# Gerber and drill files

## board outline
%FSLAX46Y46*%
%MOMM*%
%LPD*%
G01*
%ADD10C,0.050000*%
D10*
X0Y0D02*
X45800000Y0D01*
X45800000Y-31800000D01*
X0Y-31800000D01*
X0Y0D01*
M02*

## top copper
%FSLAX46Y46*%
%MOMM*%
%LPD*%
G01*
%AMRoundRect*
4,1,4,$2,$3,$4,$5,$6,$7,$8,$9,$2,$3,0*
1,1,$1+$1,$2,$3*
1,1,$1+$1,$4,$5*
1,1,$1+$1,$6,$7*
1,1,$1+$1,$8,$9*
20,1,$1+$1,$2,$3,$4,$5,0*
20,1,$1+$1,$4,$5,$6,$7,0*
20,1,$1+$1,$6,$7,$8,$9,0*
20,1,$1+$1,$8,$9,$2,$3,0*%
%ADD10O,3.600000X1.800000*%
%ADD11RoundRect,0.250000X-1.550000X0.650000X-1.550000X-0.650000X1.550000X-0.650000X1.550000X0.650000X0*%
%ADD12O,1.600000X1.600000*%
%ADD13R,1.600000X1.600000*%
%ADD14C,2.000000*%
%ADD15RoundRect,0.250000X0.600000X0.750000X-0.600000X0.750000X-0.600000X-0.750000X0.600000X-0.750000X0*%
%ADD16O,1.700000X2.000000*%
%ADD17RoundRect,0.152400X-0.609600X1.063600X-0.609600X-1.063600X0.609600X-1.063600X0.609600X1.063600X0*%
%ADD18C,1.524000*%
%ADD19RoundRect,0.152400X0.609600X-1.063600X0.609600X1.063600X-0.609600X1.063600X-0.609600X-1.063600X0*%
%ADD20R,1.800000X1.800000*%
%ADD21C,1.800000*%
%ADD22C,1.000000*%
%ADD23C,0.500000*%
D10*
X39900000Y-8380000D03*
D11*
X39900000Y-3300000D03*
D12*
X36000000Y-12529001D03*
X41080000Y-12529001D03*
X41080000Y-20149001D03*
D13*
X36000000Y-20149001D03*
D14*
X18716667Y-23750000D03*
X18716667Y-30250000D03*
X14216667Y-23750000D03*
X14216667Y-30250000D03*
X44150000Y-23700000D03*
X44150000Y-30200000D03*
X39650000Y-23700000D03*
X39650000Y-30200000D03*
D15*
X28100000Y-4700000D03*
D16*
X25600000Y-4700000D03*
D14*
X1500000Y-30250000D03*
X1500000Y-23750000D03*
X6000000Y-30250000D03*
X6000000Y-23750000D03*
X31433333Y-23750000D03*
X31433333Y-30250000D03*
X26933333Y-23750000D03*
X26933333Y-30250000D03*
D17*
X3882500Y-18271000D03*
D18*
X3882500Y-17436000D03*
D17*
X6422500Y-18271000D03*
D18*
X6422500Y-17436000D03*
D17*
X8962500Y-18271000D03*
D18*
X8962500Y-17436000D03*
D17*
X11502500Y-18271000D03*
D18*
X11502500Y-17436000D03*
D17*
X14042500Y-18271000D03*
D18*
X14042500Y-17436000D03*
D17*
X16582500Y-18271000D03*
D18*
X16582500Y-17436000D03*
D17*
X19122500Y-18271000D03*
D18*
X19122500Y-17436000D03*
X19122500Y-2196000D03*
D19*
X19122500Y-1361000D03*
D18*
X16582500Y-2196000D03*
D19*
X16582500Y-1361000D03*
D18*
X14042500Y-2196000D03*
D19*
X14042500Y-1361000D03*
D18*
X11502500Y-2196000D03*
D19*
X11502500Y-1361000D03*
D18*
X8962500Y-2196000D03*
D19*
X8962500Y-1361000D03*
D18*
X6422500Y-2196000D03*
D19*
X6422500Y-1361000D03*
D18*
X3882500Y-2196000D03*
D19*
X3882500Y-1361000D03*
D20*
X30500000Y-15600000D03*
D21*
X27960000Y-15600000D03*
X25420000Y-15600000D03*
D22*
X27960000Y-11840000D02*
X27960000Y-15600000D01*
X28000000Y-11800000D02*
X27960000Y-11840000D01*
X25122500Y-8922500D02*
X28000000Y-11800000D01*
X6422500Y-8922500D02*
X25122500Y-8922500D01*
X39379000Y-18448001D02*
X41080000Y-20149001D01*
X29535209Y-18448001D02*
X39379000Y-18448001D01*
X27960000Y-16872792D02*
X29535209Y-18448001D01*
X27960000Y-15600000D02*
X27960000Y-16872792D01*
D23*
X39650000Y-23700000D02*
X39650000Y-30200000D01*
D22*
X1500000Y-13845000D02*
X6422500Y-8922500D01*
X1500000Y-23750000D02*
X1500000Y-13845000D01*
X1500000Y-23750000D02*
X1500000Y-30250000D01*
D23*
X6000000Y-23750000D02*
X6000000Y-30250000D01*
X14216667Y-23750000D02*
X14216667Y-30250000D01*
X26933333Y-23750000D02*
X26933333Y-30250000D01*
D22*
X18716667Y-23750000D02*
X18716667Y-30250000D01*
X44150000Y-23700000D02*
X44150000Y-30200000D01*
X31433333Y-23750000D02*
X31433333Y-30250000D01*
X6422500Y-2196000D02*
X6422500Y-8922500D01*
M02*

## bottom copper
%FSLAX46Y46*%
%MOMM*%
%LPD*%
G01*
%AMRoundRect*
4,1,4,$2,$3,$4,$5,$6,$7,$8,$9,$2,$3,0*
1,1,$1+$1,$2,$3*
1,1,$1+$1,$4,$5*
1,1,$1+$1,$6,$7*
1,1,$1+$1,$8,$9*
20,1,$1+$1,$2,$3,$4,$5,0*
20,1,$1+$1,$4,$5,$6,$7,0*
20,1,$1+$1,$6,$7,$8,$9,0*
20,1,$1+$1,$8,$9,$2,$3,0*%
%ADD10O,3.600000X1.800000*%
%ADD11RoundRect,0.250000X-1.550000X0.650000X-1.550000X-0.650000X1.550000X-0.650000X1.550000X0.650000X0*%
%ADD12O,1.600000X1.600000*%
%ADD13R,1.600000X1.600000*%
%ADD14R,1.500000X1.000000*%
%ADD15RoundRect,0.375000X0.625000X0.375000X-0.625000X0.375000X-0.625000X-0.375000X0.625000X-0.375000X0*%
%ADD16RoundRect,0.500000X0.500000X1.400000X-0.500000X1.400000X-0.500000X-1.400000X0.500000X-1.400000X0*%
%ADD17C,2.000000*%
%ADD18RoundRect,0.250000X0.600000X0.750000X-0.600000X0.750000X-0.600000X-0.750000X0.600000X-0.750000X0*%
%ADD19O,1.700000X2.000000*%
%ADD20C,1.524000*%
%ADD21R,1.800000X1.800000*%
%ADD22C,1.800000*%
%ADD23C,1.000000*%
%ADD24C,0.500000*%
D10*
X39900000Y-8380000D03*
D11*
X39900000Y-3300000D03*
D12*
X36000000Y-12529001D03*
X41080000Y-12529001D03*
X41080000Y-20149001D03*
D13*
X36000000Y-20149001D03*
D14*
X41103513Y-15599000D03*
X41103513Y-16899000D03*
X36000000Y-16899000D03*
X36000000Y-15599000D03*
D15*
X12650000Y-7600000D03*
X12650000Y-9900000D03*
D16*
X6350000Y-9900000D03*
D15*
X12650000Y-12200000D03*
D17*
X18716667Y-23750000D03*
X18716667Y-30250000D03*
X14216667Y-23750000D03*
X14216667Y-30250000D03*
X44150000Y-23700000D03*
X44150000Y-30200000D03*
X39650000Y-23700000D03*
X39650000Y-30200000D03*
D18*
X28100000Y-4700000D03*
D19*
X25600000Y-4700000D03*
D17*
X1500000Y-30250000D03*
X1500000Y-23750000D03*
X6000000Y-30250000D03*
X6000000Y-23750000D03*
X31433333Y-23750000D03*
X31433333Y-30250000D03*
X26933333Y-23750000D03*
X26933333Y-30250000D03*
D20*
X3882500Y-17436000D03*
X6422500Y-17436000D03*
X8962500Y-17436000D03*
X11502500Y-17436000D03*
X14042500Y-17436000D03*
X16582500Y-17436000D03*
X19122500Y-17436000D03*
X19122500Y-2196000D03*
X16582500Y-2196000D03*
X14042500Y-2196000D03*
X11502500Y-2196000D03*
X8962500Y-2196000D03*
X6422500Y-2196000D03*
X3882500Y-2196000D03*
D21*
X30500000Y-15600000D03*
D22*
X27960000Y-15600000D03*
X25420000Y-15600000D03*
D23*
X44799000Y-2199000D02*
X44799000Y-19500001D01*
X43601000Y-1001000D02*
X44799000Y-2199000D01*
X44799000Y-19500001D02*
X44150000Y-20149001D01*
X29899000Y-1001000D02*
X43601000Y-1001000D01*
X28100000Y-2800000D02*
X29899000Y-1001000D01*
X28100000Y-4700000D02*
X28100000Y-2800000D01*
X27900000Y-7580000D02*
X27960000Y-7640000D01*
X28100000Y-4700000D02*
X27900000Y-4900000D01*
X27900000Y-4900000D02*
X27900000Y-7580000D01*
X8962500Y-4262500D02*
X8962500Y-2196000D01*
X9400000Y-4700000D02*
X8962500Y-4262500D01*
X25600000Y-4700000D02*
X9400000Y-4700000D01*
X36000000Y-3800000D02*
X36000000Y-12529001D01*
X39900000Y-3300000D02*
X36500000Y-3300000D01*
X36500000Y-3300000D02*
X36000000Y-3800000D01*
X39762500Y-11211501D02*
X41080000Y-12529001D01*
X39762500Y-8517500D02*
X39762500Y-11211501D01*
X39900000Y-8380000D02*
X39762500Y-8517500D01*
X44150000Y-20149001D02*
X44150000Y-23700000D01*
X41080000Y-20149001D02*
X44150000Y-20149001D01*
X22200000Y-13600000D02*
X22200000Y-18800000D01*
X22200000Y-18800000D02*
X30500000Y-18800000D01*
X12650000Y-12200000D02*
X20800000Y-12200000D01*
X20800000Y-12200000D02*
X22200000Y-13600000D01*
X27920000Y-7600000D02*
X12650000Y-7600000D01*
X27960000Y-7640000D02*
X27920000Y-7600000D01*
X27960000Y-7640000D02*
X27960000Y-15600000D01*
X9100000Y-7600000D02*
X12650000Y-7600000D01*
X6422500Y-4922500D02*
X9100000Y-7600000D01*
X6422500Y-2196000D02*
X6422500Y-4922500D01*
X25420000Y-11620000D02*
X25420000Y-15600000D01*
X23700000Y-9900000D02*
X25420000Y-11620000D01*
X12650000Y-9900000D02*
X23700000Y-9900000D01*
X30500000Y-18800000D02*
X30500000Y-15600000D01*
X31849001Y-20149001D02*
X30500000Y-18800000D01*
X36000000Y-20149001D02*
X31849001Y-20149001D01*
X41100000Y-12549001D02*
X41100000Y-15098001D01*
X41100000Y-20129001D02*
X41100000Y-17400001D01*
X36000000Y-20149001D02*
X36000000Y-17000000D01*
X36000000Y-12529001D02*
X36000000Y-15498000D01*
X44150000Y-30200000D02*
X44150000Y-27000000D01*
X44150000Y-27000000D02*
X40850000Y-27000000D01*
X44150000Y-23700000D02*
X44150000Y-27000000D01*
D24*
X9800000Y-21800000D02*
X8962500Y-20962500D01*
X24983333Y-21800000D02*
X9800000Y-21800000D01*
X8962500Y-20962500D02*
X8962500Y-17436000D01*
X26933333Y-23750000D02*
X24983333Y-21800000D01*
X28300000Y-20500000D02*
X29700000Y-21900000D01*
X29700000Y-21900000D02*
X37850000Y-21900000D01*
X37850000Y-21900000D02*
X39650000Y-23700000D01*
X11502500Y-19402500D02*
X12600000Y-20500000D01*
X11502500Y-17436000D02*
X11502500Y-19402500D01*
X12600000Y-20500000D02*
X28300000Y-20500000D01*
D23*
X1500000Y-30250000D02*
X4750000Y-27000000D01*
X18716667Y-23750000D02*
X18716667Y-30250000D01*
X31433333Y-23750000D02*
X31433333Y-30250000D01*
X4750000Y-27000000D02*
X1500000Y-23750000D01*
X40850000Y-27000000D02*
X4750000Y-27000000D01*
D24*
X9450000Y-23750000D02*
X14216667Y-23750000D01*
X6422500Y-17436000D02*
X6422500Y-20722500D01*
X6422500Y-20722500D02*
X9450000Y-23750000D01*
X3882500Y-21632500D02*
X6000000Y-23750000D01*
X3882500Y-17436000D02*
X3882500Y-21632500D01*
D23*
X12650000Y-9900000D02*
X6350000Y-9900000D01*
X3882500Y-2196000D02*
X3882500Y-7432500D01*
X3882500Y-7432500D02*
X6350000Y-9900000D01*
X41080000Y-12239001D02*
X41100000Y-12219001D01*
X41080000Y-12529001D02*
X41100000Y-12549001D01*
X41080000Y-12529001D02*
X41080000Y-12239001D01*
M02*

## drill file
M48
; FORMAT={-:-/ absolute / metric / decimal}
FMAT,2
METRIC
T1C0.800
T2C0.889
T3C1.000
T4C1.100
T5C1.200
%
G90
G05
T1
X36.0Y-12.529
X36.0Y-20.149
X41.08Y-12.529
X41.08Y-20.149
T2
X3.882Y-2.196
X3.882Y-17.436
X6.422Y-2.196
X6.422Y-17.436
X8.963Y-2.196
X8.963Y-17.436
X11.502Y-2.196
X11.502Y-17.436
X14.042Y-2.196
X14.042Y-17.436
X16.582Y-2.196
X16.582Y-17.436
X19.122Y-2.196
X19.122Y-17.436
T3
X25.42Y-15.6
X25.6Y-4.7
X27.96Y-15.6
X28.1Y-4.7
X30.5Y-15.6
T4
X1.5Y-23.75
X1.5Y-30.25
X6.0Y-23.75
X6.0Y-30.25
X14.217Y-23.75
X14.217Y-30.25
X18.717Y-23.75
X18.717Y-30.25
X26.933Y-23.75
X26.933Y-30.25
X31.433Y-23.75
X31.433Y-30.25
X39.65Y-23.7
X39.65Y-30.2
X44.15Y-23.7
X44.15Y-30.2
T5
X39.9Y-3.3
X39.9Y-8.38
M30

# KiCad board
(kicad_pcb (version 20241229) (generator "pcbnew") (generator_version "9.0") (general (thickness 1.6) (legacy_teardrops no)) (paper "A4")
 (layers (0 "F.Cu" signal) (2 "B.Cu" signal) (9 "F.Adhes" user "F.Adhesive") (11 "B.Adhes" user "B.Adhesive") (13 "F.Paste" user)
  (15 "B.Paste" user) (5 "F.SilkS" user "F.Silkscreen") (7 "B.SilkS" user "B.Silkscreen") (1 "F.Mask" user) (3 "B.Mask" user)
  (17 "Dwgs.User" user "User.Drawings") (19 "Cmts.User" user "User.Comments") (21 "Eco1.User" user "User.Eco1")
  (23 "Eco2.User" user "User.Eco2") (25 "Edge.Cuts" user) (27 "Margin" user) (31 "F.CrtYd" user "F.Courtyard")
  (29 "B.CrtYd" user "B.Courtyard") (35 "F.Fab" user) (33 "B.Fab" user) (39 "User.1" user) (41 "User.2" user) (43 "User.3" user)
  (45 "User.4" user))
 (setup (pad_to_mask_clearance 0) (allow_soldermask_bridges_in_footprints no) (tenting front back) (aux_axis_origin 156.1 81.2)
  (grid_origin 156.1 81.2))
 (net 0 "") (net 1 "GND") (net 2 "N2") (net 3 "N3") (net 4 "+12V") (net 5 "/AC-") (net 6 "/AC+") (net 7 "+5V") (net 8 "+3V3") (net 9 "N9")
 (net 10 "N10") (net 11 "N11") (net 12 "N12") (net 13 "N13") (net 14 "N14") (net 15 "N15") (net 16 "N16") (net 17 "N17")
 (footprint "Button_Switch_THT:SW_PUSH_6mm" (layer "F.Cu") (at 174.816667 104.95 -90)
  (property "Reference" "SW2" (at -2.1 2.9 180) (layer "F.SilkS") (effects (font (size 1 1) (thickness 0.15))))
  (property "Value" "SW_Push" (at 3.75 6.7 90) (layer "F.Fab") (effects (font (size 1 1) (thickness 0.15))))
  (pad "1" thru_hole circle (at 0 0) (size 2 2) (drill 1.1) (layers "*.Cu" "*.Mask") (remove_unused_layers no) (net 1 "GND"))
  (pad "1" thru_hole circle (at 6.5 0) (size 2 2) (drill 1.1) (layers "*.Cu" "*.Mask") (remove_unused_layers no) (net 1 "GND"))
  (pad "2" thru_hole circle (at 0 4.5) (size 2 2) (drill 1.1) (layers "*.Cu" "*.Mask") (remove_unused_layers no) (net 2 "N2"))
  (pad "2" thru_hole circle (at 6.5 4.5) (size 2 2) (drill 1.1) (layers "*.Cu" "*.Mask") (remove_unused_layers no) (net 2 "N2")))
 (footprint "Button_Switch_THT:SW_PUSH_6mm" (layer "F.Cu") (at 200.25 104.9 -90)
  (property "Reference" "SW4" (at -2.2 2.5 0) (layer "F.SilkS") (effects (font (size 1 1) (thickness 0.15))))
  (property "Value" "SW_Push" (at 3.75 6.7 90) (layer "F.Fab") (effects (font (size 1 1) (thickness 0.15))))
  (pad "1" thru_hole circle (at 0 0) (size 2 2) (drill 1.1) (layers "*.Cu" "*.Mask") (remove_unused_layers no) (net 1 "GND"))
  (pad "1" thru_hole circle (at 6.5 0) (size 2 2) (drill 1.1) (layers "*.Cu" "*.Mask") (remove_unused_layers no) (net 1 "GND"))
  (pad "2" thru_hole circle (at 0 4.5) (size 2 2) (drill 1.1) (layers "*.Cu" "*.Mask") (remove_unused_layers no) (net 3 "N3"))
  (pad "2" thru_hole circle (at 6.5 4.5) (size 2 2) (drill 1.1) (layers "*.Cu" "*.Mask") (remove_unused_layers no) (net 3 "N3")))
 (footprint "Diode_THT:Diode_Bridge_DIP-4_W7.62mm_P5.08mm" (layer "F.Cu") (at 192.1 101.349001 90)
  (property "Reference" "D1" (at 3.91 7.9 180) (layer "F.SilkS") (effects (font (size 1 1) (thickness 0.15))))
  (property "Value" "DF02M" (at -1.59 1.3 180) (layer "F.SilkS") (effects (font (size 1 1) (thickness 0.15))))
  (pad "1" thru_hole rect (at 0 0 90) (size 1.6 1.6) (drill 0.8) (layers "*.Cu" "*.Mask") (remove_unused_layers no) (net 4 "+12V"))
  (pad "2" thru_hole oval (at 0 5.08 90) (size 1.6 1.6) (drill 0.8) (layers "*.Cu" "*.Mask") (remove_unused_layers no) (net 1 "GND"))
  (pad "3" thru_hole oval (at 7.62 5.08 90) (size 1.6 1.6) (drill 0.8) (layers "*.Cu" "*.Mask") (remove_unused_layers no) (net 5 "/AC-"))
  (pad "4" thru_hole oval (at 7.62 0 90) (size 1.6 1.6) (drill 0.8) (layers "*.Cu" "*.Mask") (remove_unused_layers no) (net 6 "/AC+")))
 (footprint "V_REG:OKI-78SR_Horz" (layer "F.Cu") (at 186.6 96.8 180)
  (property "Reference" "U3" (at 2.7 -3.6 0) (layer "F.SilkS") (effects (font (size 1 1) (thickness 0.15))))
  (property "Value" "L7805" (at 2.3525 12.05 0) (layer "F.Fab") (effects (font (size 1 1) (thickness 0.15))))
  (pad "1" thru_hole rect (at 0 0) (size 1.8 1.8) (drill 1) (layers "*.Cu" "*.Mask") (remove_unused_layers no) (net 4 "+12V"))
  (pad "2" thru_hole circle (at 2.54 0) (size 1.8 1.8) (drill 1) (layers "*.Cu" "*.Mask") (remove_unused_layers no) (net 1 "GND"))
  (pad "3" thru_hole circle (at 5.08 0) (size 1.8 1.8) (drill 1) (layers "*.Cu" "*.Mask") (remove_unused_layers no) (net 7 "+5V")))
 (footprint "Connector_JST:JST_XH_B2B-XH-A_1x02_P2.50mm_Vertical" (layer "F.Cu") (at 184.2 85.9 180)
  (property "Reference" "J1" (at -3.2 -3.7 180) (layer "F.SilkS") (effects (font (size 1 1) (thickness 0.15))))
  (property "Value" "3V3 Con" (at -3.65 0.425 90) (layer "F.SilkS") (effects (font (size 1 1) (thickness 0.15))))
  (pad "1" thru_hole roundrect (at 0 0 180) (size 1.7 2) (drill 1) (layers "*.Cu" "*.Mask") (remove_unused_layers no)
   (roundrect_rratio 0.147059) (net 1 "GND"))
  (pad "2" thru_hole oval (at 2.5 0 180) (size 1.7 2) (drill 1) (layers "*.Cu" "*.Mask") (remove_unused_layers no) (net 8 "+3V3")))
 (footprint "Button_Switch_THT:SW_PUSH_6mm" (layer "F.Cu") (at 157.6 111.45 90)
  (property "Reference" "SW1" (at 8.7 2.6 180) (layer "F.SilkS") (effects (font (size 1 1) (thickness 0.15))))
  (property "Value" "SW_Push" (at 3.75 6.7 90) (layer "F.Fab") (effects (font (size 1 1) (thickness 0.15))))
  (pad "1" thru_hole circle (at 0 0 180) (size 2 2) (drill 1.1) (layers "*.Cu" "*.Mask") (remove_unused_layers no) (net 1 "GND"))
  (pad "1" thru_hole circle (at 6.5 0 180) (size 2 2) (drill 1.1) (layers "*.Cu" "*.Mask") (remove_unused_layers no) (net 1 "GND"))
  (pad "2" thru_hole circle (at 0 4.5 180) (size 2 2) (drill 1.1) (layers "*.Cu" "*.Mask") (remove_unused_layers no) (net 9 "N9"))
  (pad "2" thru_hole circle (at 6.5 4.5 180) (size 2 2) (drill 1.1) (layers "*.Cu" "*.Mask") (remove_unused_layers no) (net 9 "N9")))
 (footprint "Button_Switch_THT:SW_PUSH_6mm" (layer "F.Cu") (at 187.533333 104.95 -90)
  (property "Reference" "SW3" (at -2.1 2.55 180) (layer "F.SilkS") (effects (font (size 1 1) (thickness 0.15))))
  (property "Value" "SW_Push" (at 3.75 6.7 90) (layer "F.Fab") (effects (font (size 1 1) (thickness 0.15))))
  (pad "1" thru_hole circle (at 0 0) (size 2 2) (drill 1.1) (layers "*.Cu" "*.Mask") (remove_unused_layers no) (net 1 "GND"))
  (pad "1" thru_hole circle (at 6.5 0) (size 2 2) (drill 1.1) (layers "*.Cu" "*.Mask") (remove_unused_layers no) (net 1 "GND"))
  (pad "2" thru_hole circle (at 0 4.5) (size 2 2) (drill 1.1) (layers "*.Cu" "*.Mask") (remove_unused_layers no) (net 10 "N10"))
  (pad "2" thru_hole circle (at 6.5 4.5) (size 2 2) (drill 1.1) (layers "*.Cu" "*.Mask") (remove_unused_layers no) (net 10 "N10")))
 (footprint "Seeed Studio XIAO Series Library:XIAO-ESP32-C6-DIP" (layer "F.Cu") (at 167.6025 91.016 180)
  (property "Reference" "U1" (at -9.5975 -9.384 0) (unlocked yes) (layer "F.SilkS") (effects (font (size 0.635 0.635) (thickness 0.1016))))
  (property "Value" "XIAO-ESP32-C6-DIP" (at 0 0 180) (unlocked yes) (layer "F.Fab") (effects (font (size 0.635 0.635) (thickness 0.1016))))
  (pad "1" smd roundrect (at 7.62 -8.455 270) (size 2.432 1.524) (layers "F.Cu" "F.Mask") (roundrect_rratio 0.1) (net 9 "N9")
   (thermal_bridge_angle 45))
  (pad "1" thru_hole circle (at 7.62 -7.62 270) (size 1.524 1.524) (drill 0.889) (layers "*.Cu" "*.Mask") (remove_unused_layers no)
   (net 9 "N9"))
  (pad "2" smd roundrect (at 5.08 -8.455 270) (size 2.432 1.524) (layers "F.Cu" "F.Mask") (roundrect_rratio 0.1) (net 2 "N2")
   (thermal_bridge_angle 45))
  (pad "2" thru_hole circle (at 5.08 -7.62 270) (size 1.524 1.524) (drill 0.889) (layers "*.Cu" "*.Mask") (remove_unused_layers no)
   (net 2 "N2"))
  (pad "3" smd roundrect (at 2.54 -8.455 270) (size 2.432 1.524) (layers "F.Cu" "F.Mask") (roundrect_rratio 0.1) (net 10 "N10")
   (thermal_bridge_angle 45))
  (pad "3" thru_hole circle (at 2.54 -7.62 270) (size 1.524 1.524) (drill 0.889) (layers "*.Cu" "*.Mask") (remove_unused_layers no)
   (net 10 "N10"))
  (pad "4" smd roundrect (at 0 -8.455 270) (size 2.432 1.524) (layers "F.Cu" "F.Mask") (roundrect_rratio 0.1) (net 3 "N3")
   (thermal_bridge_angle 45))
  (pad "4" thru_hole circle (at 0 -7.62 270) (size 1.524 1.524) (drill 0.889) (layers "*.Cu" "*.Mask") (remove_unused_layers no)
   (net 3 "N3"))
  (pad "5" smd roundrect (at -2.54 -8.455 270) (size 2.432 1.524) (layers "F.Cu" "F.Mask") (roundrect_rratio 0.1) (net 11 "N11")
   (thermal_bridge_angle 45))
  (pad "5" thru_hole circle (at -2.54 -7.62 270) (size 1.524 1.524) (drill 0.889) (layers "*.Cu" "*.Mask") (remove_unused_layers no)
   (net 11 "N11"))
  (pad "6" smd roundrect (at -5.08 -8.455 270) (size 2.432 1.524) (layers "F.Cu" "F.Mask") (roundrect_rratio 0.1) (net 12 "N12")
   (thermal_bridge_angle 45))
  (pad "6" thru_hole circle (at -5.08 -7.62 270) (size 1.524 1.524) (drill 0.889) (layers "*.Cu" "*.Mask") (remove_unused_layers no)
   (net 12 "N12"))
  (pad "7" smd roundrect (at -7.62 -8.455 270) (size 2.432 1.524) (layers "F.Cu" "F.Mask") (roundrect_rratio 0.1) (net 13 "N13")
   (thermal_bridge_angle 45))
  (pad "7" thru_hole circle (at -7.62 -7.62 270) (size 1.524 1.524) (drill 0.889) (layers "*.Cu" "*.Mask") (remove_unused_layers no)
   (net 13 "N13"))
  (pad "8" thru_hole circle (at -7.62 7.62 90) (size 1.524 1.524) (drill 0.889) (layers "*.Cu" "*.Mask") (remove_unused_layers no)
   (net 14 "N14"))
  (pad "8" smd roundrect (at -7.62 8.455 90) (size 2.432 1.524) (layers "F.Cu" "F.Mask") (roundrect_rratio 0.1) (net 14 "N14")
   (thermal_bridge_angle 45))
  (pad "9" thru_hole circle (at -5.08 7.62 90) (size 1.524 1.524) (drill 0.889) (layers "*.Cu" "*.Mask") (remove_unused_layers no)
   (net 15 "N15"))
  (pad "9" smd roundrect (at -5.08 8.455 90) (size 2.432 1.524) (layers "F.Cu" "F.Mask") (roundrect_rratio 0.1) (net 15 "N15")
   (thermal_bridge_angle 45))
  (pad "10" thru_hole circle (at -2.54 7.62 90) (size 1.524 1.524) (drill 0.889) (layers "*.Cu" "*.Mask") (remove_unused_layers no)
   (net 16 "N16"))
  (pad "10" smd roundrect (at -2.54 8.455 90) (size 2.432 1.524) (layers "F.Cu" "F.Mask") (roundrect_rratio 0.1) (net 16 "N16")
   (thermal_bridge_angle 45))
  (pad "11" thru_hole circle (at 0 7.62 90) (size 1.524 1.524) (drill 0.889) (layers "*.Cu" "*.Mask") (remove_unused_layers no)
   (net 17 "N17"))
  (pad "11" smd roundrect (at 0 8.455 90) (size 2.432 1.524) (layers "F.Cu" "F.Mask") (roundrect_rratio 0.1) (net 17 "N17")
   (thermal_bridge_angle 45))
  (pad "12" thru_hole circle (at 2.54 7.62 90) (size 1.524 1.524) (drill 0.889) (layers "*.Cu" "*.Mask") (remove_unused_layers no)
   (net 8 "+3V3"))
  (pad "12" smd roundrect (at 2.54 8.455 90) (size 2.432 1.524) (layers "F.Cu" "F.Mask") (roundrect_rratio 0.1) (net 8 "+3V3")
   (thermal_bridge_angle 45))
  (pad "13" thru_hole circle (at 5.08 7.62 90) (size 1.524 1.524) (drill 0.889) (layers "*.Cu" "*.Mask") (remove_unused_layers no)
   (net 1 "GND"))
  (pad "13" smd roundrect (at 5.08 8.455 90) (size 2.432 1.524) (layers "F.Cu" "F.Mask") (roundrect_rratio 0.1) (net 1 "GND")
   (thermal_bridge_angle 45))
  (pad "14" thru_hole circle (at 7.62 7.62 90) (size 1.524 1.524) (drill 0.889) (layers "*.Cu" "*.Mask") (remove_unused_layers no)
   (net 7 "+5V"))
  (pad "14" smd roundrect (at 7.62 8.455 90) (size 2.432 1.524) (layers "F.Cu" "F.Mask") (roundrect_rratio 0.1) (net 7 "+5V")
   (thermal_bridge_angle 45)))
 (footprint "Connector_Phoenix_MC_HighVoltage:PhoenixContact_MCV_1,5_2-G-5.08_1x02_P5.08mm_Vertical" (layer "F.Cu") (at 196 84.5 -90)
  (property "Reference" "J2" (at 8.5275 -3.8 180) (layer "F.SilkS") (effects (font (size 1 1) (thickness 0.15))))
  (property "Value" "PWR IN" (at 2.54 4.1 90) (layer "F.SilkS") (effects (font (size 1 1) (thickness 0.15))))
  (pad "1" thru_hole roundrect (at 0 0 270) (size 1.8 3.6) (drill 1.2) (layers "*.Cu" "*.Mask") (remove_unused_layers no)
   (roundrect_rratio 0.138889) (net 6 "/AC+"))
  (pad "2" thru_hole oval (at 5.08 0 270) (size 1.8 3.6) (drill 1.2) (layers "*.Cu" "*.Mask") (remove_unused_layers no) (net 5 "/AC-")))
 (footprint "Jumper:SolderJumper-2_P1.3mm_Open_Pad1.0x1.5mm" (layer "B.Cu") (at 192.1 97.449 -90)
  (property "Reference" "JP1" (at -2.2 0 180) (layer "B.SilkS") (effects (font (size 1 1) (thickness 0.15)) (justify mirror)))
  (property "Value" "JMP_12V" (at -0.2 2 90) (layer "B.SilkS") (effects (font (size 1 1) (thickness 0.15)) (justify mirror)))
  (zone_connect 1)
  (pad "1" smd rect (at -0.65 0 270) (size 1 1.5) (layers "B.Cu" "B.Mask") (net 6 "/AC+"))
  (pad "2" smd rect (at 0.65 0 270) (size 1 1.5) (layers "B.Cu" "B.Mask") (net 4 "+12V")))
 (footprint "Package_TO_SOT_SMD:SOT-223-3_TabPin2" (layer "B.Cu") (at 165.6 91.1 180)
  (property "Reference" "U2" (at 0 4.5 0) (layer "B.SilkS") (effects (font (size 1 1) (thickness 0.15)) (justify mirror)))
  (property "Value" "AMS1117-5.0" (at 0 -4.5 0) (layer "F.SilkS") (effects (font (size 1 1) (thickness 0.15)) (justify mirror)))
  (pad "1" smd roundrect (at -3.15 2.3 180) (size 2 1.5) (layers "B.Cu" "B.Mask" "B.Paste") (roundrect_rratio 0.25) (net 1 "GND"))
  (pad "2" smd roundrect (at -3.15 0 180) (size 2 1.5) (layers "B.Cu" "B.Mask" "B.Paste") (roundrect_rratio 0.25) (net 7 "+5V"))
  (pad "2" smd roundrect (at 3.15 0 180) (size 2 3.8) (layers "B.Cu" "B.Mask" "B.Paste") (roundrect_rratio 0.25) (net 7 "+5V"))
  (pad "3" smd roundrect (at -3.15 -2.3 180) (size 2 1.5) (layers "B.Cu" "B.Mask" "B.Paste") (roundrect_rratio 0.25) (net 4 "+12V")))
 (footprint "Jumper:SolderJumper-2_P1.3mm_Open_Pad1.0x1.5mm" (layer "B.Cu") (at 197.203513 97.449 90)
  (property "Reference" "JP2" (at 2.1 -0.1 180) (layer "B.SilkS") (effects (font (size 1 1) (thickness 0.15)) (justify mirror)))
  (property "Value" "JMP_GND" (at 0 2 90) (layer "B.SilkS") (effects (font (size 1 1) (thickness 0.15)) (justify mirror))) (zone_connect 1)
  (pad "1" smd rect (at -0.65 0 90) (size 1 1.5) (layers "B.Cu" "B.Mask") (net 1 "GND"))
  (pad "2" smd rect (at 0.65 0 90) (size 1 1.5) (layers "B.Cu" "B.Mask") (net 5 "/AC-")))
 (gr_rect (start 156.1 81.2) (end 201.9 113) (stroke (width 0.05) (type default)) (fill no) (layer "Edge.Cuts"))
 (segment (start 195.479 99.648001) (end 197.18 101.349001) (width 1) (layer "F.Cu") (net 1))
 (segment (start 157.6 95.045) (end 162.5225 90.1225) (width 1) (layer "F.Cu") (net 1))
 (segment (start 184.1 93) (end 184.06 93.04) (width 1) (layer "F.Cu") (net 1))
 (segment (start 184.06 93.04) (end 184.06 96.8) (width 1) (layer "F.Cu") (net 1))
 (segment (start 162.5225 83.396) (end 162.5225 90.1225) (width 1) (layer "F.Cu") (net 1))
 (segment (start 184.06 96.8) (end 184.06 98.072792) (width 1) (layer "F.Cu") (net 1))
 (segment (start 184.06 98.072792) (end 185.635209 99.648001) (width 1) (layer "F.Cu") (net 1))
 (segment (start 181.2225 90.1225) (end 184.1 93) (width 1) (layer "F.Cu") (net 1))
 (segment (start 200.25 104.9) (end 200.25 111.4) (width 1) (layer "F.Cu") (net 1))
 (segment (start 187.533333 104.95) (end 187.533333 111.45) (width 1) (layer "F.Cu") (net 1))
 (segment (start 157.6 104.95) (end 157.6 111.45) (width 1) (layer "F.Cu") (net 1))
 (segment (start 157.6 104.95) (end 157.6 95.045) (width 1) (layer "F.Cu") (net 1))
 (segment (start 162.5225 90.1225) (end 181.2225 90.1225) (width 1) (layer "F.Cu") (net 1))
 (segment (start 185.635209 99.648001) (end 195.479 99.648001) (width 1) (layer "F.Cu") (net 1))
 (segment (start 174.816667 104.95) (end 174.816667 111.45) (width 1) (layer "F.Cu") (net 1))
 (segment (start 200.25 108.2) (end 196.95 108.2) (width 1) (layer "B.Cu") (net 1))
 (segment (start 184 86.1) (end 184 88.78) (width 1) (layer "B.Cu") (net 1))
 (segment (start 200.899 100.700001) (end 200.25 101.349001) (width 1) (layer "B.Cu") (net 1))
 (segment (start 185.999 82.201) (end 199.701 82.201) (width 1) (layer "B.Cu") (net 1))
 (segment (start 197.18 101.349001) (end 200.25 101.349001) (width 1) (layer "B.Cu") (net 1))
 (segment (start 184 88.78) (end 184.06 88.84) (width 1) (layer "B.Cu") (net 1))
 (segment (start 184.2 85.9) (end 184.2 84) (width 1) (layer "B.Cu") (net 1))
 (segment (start 184.06 88.84) (end 184.06 96.8) (width 1) (layer "B.Cu") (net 1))
 (segment (start 160.85 108.2) (end 157.6 104.95) (width 1) (layer "B.Cu") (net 1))
 (segment (start 184.02 88.8) (end 168.75 88.8) (width 1) (layer "B.Cu") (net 1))
 (segment (start 184.2 84) (end 185.999 82.201) (width 1) (layer "B.Cu") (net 1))
 (segment (start 184.06 88.84) (end 184.02 88.8) (width 1) (layer "B.Cu") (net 1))
 (segment (start 187.533333 104.95) (end 187.533333 111.45) (width 1) (layer "B.Cu") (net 1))
 (segment (start 162.5225 86.1225) (end 165.2 88.8) (width 1) (layer "B.Cu") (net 1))
 (segment (start 199.701 82.201) (end 200.899 83.399) (width 1) (layer "B.Cu") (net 1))
 (segment (start 200.25 101.349001) (end 200.25 104.9) (width 1) (layer "B.Cu") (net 1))
 (segment (start 157.6 111.45) (end 160.85 108.2) (width 1) (layer "B.Cu") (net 1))
 (segment (start 200.25 104.9) (end 200.25 108.2) (width 1) (layer "B.Cu") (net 1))
 (segment (start 162.5225 83.396) (end 162.5225 86.1225) (width 1) (layer "B.Cu") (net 1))
 (segment (start 165.2 88.8) (end 168.75 88.8) (width 1) (layer "B.Cu") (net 1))
 (segment (start 184.2 85.9) (end 184 86.1) (width 1) (layer "B.Cu") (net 1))
 (segment (start 200.25 111.4) (end 200.25 108.2) (width 1) (layer "B.Cu") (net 1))
 (segment (start 196.95 108.2) (end 160.85 108.2) (width 1) (layer "B.Cu") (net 1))
 (segment (start 197.2 101.329001) (end 197.2 98.600001) (width 1) (layer "B.Cu") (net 1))
 (segment (start 174.816667 104.95) (end 174.816667 111.45) (width 1) (layer "B.Cu") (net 1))
 (segment (start 200.899 83.399) (end 200.899 100.700001) (width 1) (layer "B.Cu") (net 1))
 (segment (start 165.5 85.9) (end 165.0625 85.4625) (width 1) (layer "B.Cu") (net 8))
 (segment (start 181.7 85.9) (end 165.5 85.9) (width 1) (layer "B.Cu") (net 8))
 (segment (start 165.0625 85.4625) (end 165.0625 83.396) (width 1) (layer "B.Cu") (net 8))
 (segment (start 162.1 104.95) (end 162.1 111.45) (width 0.5) (layer "F.Cu") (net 9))
 (segment (start 159.9825 98.636) (end 159.9825 102.8325) (width 0.5) (layer "B.Cu") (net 9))
 (segment (start 159.9825 102.8325) (end 162.1 104.95) (width 0.5) (layer "B.Cu") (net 9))
 (segment (start 170.316667 104.95) (end 170.316667 111.45) (width 0.5) (layer "F.Cu") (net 2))
 (segment (start 165.55 104.95) (end 170.316667 104.95) (width 0.5) (layer "B.Cu") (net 2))
 (segment (start 162.5225 101.9225) (end 165.55 104.95) (width 0.5) (layer "B.Cu") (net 2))
 (segment (start 162.5225 98.636) (end 162.5225 101.9225) (width 0.5) (layer "B.Cu") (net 2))
 (segment (start 183.033333 104.95) (end 183.033333 111.45) (width 0.5) (layer "F.Cu") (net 10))
 (segment (start 165.9 103) (end 165.0625 102.1625) (width 0.5) (layer "B.Cu") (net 10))
 (segment (start 165.0625 102.1625) (end 165.0625 98.636) (width 0.5) (layer "B.Cu") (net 10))
 (segment (start 183.033333 104.95) (end 181.083333 103) (width 0.5) (layer "B.Cu") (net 10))
 (segment (start 181.083333 103) (end 165.9 103) (width 0.5) (layer "B.Cu") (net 10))
 (segment (start 195.75 104.9) (end 195.75 111.4) (width 0.5) (layer "F.Cu") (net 3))
 (segment (start 168.7 101.7) (end 184.4 101.7) (width 0.5) (layer "B.Cu") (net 3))
 (segment (start 167.6025 100.6025) (end 168.7 101.7) (width 0.5) (layer "B.Cu") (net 3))
 (segment (start 184.4 101.7) (end 185.8 103.1) (width 0.5) (layer "B.Cu") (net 3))
 (segment (start 193.95 103.1) (end 195.75 104.9) (width 0.5) (layer "B.Cu") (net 3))
 (segment (start 167.6025 98.636) (end 167.6025 100.6025) (width 0.5) (layer "B.Cu") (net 3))
 (segment (start 185.8 103.1) (end 193.95 103.1) (width 0.5) (layer "B.Cu") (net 3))
 (segment (start 176.9 93.4) (end 178.3 94.8) (width 1) (layer "B.Cu") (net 4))
 (segment (start 192.1 101.349001) (end 187.949001 101.349001) (width 1) (layer "B.Cu") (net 4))
 (segment (start 168.75 93.4) (end 176.9 93.4) (width 1) (layer "B.Cu") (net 4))
 (segment (start 187.949001 101.349001) (end 186.6 100) (width 1) (layer "B.Cu") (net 4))
 (segment (start 186.6 100) (end 186.6 96.8) (width 1) (layer "B.Cu") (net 4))
 (segment (start 178.3 94.8) (end 178.3 100) (width 1) (layer "B.Cu") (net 4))
 (segment (start 178.3 100) (end 186.6 100) (width 1) (layer "B.Cu") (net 4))
 (segment (start 192.1 101.349001) (end 192.1 98.2) (width 1) (layer "B.Cu") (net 4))
 (segment (start 168.75 91.1) (end 179.8 91.1) (width 1) (layer "B.Cu") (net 7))
 (segment (start 168.75 91.1) (end 162.45 91.1) (width 1) (layer "B.Cu") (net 7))
 (segment (start 159.9825 83.396) (end 159.9825 88.6325) (width 1) (layer "B.Cu") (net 7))
 (segment (start 181.52 92.82) (end 181.52 96.8) (width 1) (layer "B.Cu") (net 7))
 (segment (start 159.9825 88.6325) (end 162.45 91.1) (width 1) (layer "B.Cu") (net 7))
 (segment (start 179.8 91.1) (end 181.52 92.82) (width 1) (layer "B.Cu") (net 7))
 (segment (start 195.8625 92.411501) (end 197.18 93.729001) (width 1) (layer "B.Cu") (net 5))
 (segment (start 197.18 93.729001) (end 197.18 93.439001) (width 1) (layer "B.Cu") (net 5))
 (segment (start 197.2 93.749001) (end 197.2 96.298001) (width 1) (layer "B.Cu") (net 5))
 (segment (start 196 89.58) (end 195.8625 89.7175) (width 1) (layer "B.Cu") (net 5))
 (segment (start 197.18 93.729001) (end 197.2 93.749001) (width 1) (layer "B.Cu") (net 5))
 (segment (start 195.8625 89.7175) (end 195.8625 92.411501) (width 1) (layer "B.Cu") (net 5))
 (segment (start 197.18 93.439001) (end 197.2 93.419001) (width 1) (layer "B.Cu") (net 5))
 (segment (start 192.6 84.5) (end 192.1 85) (width 1) (layer "B.Cu") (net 6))
 (segment (start 192.1 85) (end 192.1 93.729001) (width 1) (layer "B.Cu") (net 6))
 (segment (start 192.1 93.729001) (end 192.1 96.698) (width 1) (layer "B.Cu") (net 6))
 (segment (start 196 84.5) (end 192.6 84.5) (width 1) (layer "B.Cu") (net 6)))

